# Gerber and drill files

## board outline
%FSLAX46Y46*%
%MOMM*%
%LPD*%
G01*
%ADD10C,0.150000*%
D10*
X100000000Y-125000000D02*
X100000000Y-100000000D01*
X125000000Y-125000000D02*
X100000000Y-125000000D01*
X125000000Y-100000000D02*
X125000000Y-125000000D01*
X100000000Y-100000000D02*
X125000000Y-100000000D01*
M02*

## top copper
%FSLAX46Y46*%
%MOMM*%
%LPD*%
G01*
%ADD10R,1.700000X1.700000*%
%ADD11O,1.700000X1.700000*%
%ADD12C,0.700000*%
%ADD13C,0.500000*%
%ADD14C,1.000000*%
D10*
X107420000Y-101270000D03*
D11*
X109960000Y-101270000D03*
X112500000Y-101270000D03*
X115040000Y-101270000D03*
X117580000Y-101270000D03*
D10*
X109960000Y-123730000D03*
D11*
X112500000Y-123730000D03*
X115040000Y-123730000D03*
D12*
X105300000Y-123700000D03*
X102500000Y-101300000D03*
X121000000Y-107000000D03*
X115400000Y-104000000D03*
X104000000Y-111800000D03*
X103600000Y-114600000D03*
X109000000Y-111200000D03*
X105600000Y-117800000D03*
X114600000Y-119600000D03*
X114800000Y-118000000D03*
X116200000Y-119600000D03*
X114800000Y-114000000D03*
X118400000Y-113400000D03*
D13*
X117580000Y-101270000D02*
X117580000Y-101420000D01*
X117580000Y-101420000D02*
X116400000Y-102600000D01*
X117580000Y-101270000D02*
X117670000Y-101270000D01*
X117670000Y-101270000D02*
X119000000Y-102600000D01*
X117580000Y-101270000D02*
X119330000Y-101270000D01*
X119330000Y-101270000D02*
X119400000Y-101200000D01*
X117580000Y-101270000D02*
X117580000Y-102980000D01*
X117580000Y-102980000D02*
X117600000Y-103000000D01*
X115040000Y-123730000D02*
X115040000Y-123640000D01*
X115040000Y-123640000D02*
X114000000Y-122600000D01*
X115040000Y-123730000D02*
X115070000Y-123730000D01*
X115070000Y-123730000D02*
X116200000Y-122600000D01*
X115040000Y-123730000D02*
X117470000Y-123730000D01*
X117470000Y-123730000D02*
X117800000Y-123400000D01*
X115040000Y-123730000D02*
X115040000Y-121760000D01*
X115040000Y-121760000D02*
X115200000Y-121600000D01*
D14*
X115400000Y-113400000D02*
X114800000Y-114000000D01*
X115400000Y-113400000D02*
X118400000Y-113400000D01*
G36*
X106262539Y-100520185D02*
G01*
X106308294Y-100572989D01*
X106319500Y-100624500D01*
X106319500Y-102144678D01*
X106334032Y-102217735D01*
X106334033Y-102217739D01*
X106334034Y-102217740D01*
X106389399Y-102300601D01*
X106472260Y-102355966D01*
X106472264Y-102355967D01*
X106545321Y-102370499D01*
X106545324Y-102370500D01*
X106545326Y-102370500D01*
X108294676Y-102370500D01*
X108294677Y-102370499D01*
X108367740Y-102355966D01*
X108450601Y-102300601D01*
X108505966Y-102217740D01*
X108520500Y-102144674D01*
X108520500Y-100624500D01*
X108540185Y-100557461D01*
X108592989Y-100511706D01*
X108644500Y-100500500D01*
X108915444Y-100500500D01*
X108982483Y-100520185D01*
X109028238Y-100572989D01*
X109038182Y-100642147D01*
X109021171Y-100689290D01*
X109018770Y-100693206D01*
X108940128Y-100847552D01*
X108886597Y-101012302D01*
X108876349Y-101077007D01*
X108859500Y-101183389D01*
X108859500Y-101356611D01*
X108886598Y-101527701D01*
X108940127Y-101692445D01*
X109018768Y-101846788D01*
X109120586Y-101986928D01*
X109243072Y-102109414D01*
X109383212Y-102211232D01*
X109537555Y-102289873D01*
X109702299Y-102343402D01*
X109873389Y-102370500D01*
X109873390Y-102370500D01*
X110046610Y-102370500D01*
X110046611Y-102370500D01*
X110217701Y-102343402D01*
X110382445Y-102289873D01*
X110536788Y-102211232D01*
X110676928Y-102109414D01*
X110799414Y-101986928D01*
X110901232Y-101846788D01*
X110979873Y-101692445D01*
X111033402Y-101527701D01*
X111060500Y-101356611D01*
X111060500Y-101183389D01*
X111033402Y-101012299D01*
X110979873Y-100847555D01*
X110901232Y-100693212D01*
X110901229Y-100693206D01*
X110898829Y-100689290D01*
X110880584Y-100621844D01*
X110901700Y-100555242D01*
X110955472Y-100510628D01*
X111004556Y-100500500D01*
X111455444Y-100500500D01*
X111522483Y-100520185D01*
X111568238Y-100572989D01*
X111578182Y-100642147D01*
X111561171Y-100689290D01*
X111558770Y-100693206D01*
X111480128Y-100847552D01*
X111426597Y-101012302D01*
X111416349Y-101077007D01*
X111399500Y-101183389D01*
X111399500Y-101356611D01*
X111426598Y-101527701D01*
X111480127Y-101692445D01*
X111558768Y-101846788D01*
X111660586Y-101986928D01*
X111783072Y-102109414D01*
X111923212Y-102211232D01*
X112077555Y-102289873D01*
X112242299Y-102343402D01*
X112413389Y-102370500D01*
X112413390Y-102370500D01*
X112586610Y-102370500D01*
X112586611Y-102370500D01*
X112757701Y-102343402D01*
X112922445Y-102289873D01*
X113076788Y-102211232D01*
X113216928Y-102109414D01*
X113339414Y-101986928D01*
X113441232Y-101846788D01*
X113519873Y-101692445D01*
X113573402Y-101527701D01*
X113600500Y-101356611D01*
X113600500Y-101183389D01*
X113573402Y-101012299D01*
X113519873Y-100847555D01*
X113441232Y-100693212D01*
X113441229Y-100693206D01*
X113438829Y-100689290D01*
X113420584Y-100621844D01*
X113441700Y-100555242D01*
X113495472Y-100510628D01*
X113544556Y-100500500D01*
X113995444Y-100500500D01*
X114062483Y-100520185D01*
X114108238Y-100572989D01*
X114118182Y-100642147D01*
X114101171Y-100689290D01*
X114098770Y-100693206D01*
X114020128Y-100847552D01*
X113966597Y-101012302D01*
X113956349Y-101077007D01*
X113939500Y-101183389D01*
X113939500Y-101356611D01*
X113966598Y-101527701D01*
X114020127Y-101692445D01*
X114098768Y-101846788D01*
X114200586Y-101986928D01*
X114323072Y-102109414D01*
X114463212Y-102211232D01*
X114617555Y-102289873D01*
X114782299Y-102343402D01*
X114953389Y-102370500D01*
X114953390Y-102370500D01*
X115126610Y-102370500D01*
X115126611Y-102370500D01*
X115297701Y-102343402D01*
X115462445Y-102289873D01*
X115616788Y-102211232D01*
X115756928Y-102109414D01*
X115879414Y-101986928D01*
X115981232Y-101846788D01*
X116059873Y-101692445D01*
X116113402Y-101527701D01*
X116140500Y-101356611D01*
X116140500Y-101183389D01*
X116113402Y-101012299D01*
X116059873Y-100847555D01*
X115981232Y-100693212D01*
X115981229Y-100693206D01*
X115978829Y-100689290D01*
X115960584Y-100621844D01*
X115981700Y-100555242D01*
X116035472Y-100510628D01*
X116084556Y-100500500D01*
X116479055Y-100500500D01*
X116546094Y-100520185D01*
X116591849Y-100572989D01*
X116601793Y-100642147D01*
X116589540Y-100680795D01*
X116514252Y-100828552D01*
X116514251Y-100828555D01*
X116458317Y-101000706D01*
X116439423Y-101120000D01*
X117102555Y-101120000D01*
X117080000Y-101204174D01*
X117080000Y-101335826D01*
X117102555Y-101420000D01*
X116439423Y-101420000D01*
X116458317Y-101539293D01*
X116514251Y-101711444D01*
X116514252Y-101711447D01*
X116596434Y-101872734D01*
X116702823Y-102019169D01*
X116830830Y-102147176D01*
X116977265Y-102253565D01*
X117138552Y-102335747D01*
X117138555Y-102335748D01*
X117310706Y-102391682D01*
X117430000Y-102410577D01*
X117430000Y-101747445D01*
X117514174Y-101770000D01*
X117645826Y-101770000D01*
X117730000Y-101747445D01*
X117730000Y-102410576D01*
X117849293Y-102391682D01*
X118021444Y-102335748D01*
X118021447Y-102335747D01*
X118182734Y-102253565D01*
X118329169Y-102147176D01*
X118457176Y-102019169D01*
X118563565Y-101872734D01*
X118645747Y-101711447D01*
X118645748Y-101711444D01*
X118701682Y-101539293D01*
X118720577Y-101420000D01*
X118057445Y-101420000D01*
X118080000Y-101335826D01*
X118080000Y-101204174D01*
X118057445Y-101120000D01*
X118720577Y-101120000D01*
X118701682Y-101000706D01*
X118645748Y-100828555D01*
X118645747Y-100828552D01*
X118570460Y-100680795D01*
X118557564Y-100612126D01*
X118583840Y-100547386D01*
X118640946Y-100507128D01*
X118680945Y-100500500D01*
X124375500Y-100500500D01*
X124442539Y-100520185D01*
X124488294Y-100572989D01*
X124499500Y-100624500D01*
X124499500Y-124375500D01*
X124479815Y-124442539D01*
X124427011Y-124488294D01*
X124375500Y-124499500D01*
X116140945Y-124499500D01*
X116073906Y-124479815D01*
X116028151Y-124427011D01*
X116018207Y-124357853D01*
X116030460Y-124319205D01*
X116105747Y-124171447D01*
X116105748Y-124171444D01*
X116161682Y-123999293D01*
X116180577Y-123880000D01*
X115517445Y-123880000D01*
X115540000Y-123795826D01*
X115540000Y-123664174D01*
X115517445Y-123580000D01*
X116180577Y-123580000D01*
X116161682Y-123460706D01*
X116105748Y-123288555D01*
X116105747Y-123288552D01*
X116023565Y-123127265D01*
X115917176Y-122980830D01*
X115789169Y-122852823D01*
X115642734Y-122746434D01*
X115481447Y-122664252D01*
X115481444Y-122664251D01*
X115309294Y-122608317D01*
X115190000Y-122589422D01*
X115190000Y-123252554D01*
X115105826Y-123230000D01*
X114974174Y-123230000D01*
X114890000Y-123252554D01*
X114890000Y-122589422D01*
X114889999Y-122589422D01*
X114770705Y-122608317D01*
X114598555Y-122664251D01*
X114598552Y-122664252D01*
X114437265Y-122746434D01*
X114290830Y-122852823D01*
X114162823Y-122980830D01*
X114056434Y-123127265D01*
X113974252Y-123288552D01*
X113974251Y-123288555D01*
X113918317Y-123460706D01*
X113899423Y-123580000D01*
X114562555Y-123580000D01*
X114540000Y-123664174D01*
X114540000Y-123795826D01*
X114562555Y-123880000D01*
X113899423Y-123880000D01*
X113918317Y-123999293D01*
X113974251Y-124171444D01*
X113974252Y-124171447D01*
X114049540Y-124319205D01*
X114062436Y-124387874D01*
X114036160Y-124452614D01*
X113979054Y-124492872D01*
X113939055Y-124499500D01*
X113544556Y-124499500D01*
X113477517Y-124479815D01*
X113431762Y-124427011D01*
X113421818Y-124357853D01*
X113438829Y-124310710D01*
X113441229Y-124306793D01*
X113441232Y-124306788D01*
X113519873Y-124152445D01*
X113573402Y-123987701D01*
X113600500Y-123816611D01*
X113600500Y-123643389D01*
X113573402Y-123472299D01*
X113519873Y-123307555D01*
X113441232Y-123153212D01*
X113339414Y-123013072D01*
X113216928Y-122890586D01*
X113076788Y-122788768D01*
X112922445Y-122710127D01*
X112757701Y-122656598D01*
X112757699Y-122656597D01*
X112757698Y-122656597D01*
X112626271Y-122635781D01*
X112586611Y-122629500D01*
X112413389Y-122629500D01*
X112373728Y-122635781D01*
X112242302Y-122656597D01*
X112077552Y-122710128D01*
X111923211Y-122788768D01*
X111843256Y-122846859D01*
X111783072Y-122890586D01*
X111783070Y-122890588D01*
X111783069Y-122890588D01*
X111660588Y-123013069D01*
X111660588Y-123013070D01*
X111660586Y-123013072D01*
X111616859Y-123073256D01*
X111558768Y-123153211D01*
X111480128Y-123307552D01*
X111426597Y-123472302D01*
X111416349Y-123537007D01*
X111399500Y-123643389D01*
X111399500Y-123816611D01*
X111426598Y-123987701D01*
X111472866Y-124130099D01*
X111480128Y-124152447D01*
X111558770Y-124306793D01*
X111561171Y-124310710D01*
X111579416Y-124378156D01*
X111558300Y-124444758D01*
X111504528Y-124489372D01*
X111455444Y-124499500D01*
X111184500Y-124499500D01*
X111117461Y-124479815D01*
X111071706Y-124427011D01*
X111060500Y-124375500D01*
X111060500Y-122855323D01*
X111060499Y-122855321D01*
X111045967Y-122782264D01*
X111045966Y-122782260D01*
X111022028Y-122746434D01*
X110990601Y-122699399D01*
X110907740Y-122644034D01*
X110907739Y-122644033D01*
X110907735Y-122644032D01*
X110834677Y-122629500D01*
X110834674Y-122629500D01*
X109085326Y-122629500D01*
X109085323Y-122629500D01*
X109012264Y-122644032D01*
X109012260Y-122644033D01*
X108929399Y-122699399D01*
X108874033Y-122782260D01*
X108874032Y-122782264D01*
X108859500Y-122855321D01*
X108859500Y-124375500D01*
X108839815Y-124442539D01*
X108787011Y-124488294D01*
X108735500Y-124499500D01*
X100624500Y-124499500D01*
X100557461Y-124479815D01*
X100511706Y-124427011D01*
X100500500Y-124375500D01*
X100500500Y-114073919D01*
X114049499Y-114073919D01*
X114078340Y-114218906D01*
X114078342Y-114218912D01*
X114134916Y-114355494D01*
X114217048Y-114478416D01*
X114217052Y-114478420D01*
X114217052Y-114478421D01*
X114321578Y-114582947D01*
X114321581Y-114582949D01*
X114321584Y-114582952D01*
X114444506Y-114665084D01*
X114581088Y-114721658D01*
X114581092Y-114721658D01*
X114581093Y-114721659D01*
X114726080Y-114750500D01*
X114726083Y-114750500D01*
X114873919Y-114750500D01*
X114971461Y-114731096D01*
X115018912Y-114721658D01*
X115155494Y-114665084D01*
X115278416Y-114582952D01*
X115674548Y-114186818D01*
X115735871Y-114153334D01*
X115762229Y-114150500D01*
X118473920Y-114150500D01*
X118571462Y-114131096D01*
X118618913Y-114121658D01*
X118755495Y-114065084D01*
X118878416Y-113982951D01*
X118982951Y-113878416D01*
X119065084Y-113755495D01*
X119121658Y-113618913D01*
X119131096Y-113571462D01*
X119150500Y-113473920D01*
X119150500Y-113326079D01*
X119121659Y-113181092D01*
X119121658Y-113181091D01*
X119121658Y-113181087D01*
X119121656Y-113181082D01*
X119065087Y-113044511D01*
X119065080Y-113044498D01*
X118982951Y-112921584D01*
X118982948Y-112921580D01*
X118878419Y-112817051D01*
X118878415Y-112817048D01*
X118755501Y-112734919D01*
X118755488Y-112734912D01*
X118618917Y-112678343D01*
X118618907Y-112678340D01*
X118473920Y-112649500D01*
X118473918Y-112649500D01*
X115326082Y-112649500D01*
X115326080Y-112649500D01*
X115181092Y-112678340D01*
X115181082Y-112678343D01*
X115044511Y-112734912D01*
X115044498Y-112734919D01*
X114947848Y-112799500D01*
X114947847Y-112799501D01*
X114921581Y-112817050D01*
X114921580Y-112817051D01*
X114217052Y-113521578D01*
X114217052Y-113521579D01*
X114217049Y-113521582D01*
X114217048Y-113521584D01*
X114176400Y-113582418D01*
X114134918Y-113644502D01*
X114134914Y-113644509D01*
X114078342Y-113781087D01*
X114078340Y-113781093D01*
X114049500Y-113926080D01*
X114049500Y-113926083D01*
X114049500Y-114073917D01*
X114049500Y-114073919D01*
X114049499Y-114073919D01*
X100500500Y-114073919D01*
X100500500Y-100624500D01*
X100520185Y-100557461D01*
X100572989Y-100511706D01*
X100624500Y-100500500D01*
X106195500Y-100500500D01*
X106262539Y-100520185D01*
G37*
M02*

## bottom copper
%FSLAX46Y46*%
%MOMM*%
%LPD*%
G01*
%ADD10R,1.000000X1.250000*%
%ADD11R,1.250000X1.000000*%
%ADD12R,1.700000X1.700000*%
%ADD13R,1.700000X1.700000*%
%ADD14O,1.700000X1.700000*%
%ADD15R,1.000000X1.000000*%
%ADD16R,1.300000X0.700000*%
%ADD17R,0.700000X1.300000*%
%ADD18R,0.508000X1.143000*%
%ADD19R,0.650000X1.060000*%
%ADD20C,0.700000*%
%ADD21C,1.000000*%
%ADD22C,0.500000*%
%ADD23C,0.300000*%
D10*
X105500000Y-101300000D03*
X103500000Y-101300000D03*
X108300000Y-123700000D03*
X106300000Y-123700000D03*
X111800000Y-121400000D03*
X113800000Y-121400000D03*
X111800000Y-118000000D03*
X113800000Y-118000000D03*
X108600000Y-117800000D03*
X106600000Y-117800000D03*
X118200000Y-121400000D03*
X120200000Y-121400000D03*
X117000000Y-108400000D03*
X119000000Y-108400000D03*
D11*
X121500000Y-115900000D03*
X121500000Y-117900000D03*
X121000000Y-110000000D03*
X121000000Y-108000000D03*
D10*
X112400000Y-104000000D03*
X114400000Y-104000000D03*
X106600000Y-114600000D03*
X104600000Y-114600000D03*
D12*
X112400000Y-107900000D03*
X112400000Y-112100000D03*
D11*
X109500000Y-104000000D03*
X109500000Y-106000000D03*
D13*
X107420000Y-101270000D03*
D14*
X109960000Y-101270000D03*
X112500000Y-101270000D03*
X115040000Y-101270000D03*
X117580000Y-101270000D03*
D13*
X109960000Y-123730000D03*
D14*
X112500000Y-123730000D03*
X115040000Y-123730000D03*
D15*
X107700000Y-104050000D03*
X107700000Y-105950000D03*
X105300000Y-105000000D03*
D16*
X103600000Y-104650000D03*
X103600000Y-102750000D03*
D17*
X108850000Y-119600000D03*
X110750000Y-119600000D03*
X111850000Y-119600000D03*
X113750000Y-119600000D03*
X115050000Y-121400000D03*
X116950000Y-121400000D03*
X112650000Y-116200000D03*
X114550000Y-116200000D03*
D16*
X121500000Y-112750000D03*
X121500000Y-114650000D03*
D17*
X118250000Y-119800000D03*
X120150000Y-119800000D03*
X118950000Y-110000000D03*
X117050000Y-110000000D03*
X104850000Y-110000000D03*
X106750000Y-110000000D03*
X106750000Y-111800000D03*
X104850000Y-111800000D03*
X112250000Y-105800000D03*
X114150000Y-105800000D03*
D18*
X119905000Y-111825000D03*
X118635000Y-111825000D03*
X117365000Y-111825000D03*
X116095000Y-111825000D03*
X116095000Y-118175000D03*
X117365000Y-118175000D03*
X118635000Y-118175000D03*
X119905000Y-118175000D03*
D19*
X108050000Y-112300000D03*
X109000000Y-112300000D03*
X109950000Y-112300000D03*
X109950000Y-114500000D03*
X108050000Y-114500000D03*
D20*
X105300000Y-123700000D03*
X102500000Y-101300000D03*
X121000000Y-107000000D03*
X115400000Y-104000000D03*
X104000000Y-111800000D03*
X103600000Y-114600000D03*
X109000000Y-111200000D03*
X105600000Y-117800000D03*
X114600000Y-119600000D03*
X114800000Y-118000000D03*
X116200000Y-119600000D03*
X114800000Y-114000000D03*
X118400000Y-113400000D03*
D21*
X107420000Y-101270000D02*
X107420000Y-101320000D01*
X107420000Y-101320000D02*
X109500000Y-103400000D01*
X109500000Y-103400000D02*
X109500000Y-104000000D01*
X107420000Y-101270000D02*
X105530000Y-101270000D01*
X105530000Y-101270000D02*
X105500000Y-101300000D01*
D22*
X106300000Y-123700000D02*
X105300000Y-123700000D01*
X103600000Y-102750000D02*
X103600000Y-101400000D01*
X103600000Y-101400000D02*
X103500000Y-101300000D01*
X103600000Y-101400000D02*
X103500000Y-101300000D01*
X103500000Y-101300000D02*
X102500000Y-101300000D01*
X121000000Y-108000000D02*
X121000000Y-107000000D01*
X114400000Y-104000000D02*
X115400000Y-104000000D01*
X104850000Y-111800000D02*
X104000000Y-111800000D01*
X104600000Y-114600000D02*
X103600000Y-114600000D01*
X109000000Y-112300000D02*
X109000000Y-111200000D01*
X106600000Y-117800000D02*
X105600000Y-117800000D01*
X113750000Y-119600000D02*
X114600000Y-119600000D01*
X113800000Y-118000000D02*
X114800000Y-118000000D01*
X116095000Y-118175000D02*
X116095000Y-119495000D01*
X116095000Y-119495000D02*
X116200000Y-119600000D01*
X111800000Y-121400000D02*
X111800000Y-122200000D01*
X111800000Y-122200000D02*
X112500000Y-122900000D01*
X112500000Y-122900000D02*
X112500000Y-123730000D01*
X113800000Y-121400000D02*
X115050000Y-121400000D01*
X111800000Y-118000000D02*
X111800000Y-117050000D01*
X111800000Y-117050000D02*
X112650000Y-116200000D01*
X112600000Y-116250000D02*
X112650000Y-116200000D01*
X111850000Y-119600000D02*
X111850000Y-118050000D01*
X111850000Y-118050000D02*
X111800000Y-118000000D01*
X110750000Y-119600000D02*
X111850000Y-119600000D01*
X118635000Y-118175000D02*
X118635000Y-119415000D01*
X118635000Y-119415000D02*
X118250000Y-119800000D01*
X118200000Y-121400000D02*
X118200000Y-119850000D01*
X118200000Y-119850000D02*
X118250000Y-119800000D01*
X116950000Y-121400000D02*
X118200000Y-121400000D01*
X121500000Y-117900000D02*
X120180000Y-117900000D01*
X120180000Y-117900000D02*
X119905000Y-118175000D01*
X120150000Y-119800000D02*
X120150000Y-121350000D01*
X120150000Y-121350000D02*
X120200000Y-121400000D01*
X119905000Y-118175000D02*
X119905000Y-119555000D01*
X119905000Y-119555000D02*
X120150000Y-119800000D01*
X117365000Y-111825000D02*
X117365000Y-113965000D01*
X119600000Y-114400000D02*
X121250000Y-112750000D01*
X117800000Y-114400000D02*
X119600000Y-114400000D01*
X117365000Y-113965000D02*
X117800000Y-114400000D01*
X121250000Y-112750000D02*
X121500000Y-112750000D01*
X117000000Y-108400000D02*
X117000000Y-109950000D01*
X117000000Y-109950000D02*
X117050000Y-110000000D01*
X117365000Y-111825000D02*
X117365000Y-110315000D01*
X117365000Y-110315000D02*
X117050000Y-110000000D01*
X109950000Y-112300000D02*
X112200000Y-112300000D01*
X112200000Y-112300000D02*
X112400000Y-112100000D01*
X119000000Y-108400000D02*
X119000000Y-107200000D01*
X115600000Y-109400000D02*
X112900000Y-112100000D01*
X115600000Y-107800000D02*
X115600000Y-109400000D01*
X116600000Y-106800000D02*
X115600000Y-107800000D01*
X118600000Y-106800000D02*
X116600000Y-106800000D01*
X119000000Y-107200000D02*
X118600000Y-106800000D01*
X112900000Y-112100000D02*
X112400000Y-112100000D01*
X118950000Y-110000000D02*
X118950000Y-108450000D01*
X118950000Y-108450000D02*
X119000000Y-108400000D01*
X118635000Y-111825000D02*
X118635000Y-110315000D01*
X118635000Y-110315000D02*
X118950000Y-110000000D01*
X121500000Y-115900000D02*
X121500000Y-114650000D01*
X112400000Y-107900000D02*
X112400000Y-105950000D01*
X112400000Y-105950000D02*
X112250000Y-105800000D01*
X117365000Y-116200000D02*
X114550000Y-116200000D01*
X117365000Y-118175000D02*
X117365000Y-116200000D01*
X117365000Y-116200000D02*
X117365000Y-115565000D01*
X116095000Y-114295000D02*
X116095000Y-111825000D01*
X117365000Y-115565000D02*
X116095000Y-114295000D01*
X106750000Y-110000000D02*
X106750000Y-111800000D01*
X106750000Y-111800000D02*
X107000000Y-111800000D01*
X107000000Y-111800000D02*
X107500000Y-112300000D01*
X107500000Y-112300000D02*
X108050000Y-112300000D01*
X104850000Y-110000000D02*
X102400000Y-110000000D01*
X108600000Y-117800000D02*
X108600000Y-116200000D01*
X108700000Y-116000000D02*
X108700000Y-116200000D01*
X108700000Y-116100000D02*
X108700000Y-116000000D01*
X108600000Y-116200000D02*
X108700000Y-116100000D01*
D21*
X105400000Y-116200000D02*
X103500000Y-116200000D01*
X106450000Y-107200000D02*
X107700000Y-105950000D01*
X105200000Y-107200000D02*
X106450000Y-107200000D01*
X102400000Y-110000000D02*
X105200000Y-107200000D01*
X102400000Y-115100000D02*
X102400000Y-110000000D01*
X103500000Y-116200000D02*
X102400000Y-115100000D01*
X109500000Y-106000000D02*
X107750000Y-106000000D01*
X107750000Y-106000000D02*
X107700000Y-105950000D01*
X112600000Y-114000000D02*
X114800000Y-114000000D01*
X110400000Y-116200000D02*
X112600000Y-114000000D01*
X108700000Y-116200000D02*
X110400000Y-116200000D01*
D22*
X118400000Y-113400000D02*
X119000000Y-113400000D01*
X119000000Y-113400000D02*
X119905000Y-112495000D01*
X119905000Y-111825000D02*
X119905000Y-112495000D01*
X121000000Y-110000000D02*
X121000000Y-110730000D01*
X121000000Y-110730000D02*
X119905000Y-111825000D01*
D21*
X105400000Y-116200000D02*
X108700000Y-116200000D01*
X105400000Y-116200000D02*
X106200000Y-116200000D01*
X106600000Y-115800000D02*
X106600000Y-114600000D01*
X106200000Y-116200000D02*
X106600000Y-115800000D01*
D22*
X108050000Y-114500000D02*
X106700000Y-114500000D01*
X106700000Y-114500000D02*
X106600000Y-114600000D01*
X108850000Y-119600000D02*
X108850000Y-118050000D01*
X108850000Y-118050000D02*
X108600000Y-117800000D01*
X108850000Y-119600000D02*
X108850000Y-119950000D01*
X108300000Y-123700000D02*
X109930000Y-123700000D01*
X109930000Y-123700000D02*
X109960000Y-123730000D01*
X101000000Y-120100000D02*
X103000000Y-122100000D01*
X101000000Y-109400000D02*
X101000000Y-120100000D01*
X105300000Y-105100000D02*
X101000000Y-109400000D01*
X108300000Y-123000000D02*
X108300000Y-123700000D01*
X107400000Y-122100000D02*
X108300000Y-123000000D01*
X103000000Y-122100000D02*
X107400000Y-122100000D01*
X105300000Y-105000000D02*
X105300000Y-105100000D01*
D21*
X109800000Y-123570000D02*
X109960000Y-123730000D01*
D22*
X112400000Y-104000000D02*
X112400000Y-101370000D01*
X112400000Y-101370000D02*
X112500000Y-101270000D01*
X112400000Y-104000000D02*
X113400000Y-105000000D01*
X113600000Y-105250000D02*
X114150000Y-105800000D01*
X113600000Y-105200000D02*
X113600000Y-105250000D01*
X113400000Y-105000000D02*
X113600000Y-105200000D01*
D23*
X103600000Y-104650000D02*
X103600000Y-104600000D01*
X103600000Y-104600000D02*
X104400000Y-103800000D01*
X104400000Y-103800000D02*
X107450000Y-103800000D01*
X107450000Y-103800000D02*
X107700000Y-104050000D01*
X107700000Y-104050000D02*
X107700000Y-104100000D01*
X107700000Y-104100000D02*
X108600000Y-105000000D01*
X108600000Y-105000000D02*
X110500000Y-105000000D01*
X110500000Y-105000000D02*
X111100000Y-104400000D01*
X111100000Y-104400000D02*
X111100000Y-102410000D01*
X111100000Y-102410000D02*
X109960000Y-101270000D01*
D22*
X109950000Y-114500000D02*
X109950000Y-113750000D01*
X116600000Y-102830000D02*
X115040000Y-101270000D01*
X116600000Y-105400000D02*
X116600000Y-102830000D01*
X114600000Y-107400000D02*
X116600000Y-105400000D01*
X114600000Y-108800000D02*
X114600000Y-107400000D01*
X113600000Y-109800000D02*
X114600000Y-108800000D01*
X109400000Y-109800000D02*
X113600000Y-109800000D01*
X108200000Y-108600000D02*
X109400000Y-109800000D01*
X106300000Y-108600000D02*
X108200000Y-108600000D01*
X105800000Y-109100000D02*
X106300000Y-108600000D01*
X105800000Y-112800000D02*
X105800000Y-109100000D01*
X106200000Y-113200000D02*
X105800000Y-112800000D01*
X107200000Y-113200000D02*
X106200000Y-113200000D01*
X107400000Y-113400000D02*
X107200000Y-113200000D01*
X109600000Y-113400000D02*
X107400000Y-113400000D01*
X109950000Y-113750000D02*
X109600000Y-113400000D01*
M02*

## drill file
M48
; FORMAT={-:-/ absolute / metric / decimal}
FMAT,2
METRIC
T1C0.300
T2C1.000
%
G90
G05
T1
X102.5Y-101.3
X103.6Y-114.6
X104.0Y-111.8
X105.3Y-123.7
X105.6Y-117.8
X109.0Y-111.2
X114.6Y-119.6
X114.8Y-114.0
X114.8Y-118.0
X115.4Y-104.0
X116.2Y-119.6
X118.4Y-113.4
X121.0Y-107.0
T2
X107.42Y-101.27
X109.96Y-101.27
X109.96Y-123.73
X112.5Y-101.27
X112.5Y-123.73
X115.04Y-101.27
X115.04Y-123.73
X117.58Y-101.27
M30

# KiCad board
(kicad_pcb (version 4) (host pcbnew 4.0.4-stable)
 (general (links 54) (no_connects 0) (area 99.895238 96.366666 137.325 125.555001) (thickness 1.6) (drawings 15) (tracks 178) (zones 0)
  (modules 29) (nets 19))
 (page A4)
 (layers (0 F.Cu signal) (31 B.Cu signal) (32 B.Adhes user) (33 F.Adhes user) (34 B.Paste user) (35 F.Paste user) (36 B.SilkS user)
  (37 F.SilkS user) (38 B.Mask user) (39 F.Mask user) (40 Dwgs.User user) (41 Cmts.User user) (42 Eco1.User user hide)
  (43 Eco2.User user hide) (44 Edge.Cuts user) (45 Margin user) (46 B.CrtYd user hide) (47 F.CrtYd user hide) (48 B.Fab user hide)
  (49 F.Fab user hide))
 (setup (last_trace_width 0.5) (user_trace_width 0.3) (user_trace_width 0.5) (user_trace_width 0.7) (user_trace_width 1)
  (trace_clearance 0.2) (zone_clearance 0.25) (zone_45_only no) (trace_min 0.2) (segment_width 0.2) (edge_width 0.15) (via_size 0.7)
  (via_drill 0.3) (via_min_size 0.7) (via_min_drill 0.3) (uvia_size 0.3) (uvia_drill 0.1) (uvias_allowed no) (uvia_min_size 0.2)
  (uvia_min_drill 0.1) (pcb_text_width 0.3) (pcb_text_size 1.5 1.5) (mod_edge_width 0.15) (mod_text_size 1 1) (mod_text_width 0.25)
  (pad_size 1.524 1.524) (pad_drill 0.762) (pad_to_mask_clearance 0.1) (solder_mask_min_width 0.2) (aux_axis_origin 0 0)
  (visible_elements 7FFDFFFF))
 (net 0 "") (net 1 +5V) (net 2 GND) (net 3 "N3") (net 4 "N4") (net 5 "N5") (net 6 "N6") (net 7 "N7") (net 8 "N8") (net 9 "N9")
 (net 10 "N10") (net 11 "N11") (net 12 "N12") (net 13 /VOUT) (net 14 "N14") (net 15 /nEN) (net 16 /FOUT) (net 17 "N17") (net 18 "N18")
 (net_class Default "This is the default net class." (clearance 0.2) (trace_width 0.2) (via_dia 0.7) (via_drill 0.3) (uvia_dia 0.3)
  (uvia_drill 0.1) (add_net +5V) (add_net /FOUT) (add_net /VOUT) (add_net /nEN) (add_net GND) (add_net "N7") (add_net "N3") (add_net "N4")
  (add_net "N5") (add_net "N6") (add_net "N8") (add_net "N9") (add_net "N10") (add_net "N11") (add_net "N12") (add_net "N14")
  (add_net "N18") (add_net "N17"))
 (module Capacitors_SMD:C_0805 (layer B.Cu) (at 104.5 101.3 180)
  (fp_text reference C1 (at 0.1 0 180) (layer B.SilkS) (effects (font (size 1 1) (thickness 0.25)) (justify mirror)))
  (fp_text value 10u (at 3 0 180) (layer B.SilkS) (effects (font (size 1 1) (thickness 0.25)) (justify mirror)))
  (pad 1 smd rect (at -1 0 180) (size 1 1.25) (layers B.Cu B.Paste B.Mask) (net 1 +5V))
  (pad 2 smd rect (at 1 0 180) (size 1 1.25) (layers B.Cu B.Paste B.Mask) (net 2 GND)))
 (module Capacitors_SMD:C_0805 (layer B.Cu) (at 107.3 123.7 180)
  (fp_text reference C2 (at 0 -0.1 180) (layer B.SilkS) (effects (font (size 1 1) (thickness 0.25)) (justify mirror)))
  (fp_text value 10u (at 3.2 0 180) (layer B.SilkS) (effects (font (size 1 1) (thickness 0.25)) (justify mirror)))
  (pad 1 smd rect (at -1 0 180) (size 1 1.25) (layers B.Cu B.Paste B.Mask) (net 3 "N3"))
  (pad 2 smd rect (at 1 0 180) (size 1 1.25) (layers B.Cu B.Paste B.Mask) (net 2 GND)))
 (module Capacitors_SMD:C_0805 (layer B.Cu) (at 112.8 121.4)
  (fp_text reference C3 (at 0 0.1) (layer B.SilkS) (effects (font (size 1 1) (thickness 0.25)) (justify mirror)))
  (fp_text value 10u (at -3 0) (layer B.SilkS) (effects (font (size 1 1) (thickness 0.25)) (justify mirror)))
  (pad 1 smd rect (at -1 0) (size 1 1.25) (layers B.Cu B.Paste B.Mask) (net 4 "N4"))
  (pad 2 smd rect (at 1 0) (size 1 1.25) (layers B.Cu B.Paste B.Mask) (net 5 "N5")))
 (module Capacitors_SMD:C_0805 (layer B.Cu) (at 112.8 118)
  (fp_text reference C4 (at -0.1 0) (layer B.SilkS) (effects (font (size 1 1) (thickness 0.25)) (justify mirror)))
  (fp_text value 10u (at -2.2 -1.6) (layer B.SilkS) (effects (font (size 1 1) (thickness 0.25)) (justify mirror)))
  (pad 1 smd rect (at -1 0) (size 1 1.25) (layers B.Cu B.Paste B.Mask) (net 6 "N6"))
  (pad 2 smd rect (at 1 0) (size 1 1.25) (layers B.Cu B.Paste B.Mask) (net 2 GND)))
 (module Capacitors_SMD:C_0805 (layer B.Cu) (at 107.6 117.8 180)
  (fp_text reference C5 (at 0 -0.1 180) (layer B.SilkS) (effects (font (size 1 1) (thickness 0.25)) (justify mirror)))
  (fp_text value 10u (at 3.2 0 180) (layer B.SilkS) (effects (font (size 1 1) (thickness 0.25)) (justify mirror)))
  (pad 1 smd rect (at -1 0 180) (size 1 1.25) (layers B.Cu B.Paste B.Mask) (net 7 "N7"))
  (pad 2 smd rect (at 1 0 180) (size 1 1.25) (layers B.Cu B.Paste B.Mask) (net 2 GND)))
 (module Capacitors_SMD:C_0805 (layer B.Cu) (at 119.2 121.4)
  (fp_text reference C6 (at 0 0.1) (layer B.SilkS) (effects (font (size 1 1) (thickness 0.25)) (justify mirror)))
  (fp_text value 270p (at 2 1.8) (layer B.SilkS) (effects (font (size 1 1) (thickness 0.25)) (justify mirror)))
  (pad 1 smd rect (at -1 0) (size 1 1.25) (layers B.Cu B.Paste B.Mask) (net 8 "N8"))
  (pad 2 smd rect (at 1 0) (size 1 1.25) (layers B.Cu B.Paste B.Mask) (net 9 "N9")))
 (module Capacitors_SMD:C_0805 (layer B.Cu) (at 118 108.4)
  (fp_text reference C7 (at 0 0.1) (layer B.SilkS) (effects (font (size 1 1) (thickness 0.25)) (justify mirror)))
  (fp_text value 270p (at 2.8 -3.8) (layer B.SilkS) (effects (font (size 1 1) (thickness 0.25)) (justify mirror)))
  (pad 1 smd rect (at -1 0) (size 1 1.25) (layers B.Cu B.Paste B.Mask) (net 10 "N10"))
  (pad 2 smd rect (at 1 0) (size 1 1.25) (layers B.Cu B.Paste B.Mask) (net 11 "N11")))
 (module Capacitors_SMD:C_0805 (layer B.Cu) (at 121.5 116.9 270)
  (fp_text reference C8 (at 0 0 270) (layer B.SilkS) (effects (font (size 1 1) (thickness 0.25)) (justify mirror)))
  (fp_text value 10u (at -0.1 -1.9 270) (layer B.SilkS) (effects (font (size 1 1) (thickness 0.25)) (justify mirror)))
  (pad 1 smd rect (at -1 0 270) (size 1 1.25) (layers B.Cu B.Paste B.Mask) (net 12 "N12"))
  (pad 2 smd rect (at 1 0 270) (size 1 1.25) (layers B.Cu B.Paste B.Mask) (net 9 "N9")))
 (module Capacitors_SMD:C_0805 (layer B.Cu) (at 121 109 90)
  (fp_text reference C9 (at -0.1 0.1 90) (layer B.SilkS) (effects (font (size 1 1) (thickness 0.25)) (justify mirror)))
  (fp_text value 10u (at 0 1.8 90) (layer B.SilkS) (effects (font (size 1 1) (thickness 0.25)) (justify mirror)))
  (pad 1 smd rect (at -1 0 90) (size 1 1.25) (layers B.Cu B.Paste B.Mask) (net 7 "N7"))
  (pad 2 smd rect (at 1 0 90) (size 1 1.25) (layers B.Cu B.Paste B.Mask) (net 2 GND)))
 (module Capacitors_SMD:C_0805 (layer B.Cu) (at 113.4 104)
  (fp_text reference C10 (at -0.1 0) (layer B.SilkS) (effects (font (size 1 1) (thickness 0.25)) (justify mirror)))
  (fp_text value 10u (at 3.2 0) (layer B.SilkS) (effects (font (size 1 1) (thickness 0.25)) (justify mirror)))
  (pad 1 smd rect (at -1 0) (size 1 1.25) (layers B.Cu B.Paste B.Mask) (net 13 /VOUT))
  (pad 2 smd rect (at 1 0) (size 1 1.25) (layers B.Cu B.Paste B.Mask) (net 2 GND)))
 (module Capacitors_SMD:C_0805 (layer B.Cu) (at 105.6 114.6 180)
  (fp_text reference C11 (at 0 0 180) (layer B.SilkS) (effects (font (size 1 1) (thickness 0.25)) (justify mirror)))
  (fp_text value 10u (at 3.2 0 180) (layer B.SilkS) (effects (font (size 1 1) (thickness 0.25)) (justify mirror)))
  (pad 1 smd rect (at -1 0 180) (size 1 1.25) (layers B.Cu B.Paste B.Mask) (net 7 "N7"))
  (pad 2 smd rect (at 1 0 180) (size 1 1.25) (layers B.Cu B.Paste B.Mask) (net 2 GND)))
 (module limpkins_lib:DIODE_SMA (layer B.Cu) (at 112.4 110 270)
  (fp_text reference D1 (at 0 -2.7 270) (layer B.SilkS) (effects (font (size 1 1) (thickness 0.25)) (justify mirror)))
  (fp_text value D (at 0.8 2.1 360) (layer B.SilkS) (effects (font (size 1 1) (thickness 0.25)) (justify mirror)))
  (pad 1 smd rect (at -2.1 0 270) (size 1.7 1.7) (layers B.Cu B.Paste B.Mask) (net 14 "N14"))
  (pad 2 smd rect (at 2.1 0 270) (size 1.7 1.7) (layers B.Cu B.Paste B.Mask) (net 11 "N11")))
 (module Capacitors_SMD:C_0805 (layer B.Cu) (at 109.5 105 270)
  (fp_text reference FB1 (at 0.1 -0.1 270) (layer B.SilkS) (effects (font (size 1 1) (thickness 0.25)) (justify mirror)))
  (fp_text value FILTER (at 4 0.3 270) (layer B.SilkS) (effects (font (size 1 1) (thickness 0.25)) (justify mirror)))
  (pad 1 smd rect (at -1 0 270) (size 1 1.25) (layers B.Cu B.Paste B.Mask) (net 1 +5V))
  (pad 2 smd rect (at 1 0 270) (size 1 1.25) (layers B.Cu B.Paste B.Mask) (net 7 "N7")))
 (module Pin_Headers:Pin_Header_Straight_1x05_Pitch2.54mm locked (layer F.Cu) (at 107.42 101.27 90)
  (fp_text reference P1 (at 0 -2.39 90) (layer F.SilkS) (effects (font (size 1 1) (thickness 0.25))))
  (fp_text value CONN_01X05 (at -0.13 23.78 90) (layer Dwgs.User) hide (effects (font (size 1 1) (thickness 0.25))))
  (pad 1 thru_hole rect (at 0 0 90) (size 1.7 1.7) (drill 1) (layers *.Cu *.Mask) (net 1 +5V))
  (pad 2 thru_hole oval (at 0 2.54 90) (size 1.7 1.7) (drill 1) (layers *.Cu *.Mask) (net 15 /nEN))
  (pad 3 thru_hole oval (at 0 5.08 90) (size 1.7 1.7) (drill 1) (layers *.Cu *.Mask) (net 13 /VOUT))
  (pad 4 thru_hole oval (at 0 7.62 90) (size 1.7 1.7) (drill 1) (layers *.Cu *.Mask) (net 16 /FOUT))
  (pad 5 thru_hole oval (at 0 10.16 90) (size 1.7 1.7) (drill 1) (layers *.Cu *.Mask) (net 2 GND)))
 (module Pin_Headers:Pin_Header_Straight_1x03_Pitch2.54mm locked (layer F.Cu) (at 109.96 123.73 90)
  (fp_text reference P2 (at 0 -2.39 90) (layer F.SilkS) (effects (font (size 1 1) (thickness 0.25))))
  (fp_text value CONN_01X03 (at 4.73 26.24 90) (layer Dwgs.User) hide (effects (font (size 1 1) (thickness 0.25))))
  (pad 1 thru_hole rect (at 0 0 90) (size 1.7 1.7) (drill 1) (layers *.Cu *.Mask) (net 3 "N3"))
  (pad 2 thru_hole oval (at 0 2.54 90) (size 1.7 1.7) (drill 1) (layers *.Cu *.Mask) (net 4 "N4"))
  (pad 3 thru_hole oval (at 0 5.08 90) (size 1.7 1.7) (drill 1) (layers *.Cu *.Mask) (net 2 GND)))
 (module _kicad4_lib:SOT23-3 (layer B.Cu) (at 106.5 105 270)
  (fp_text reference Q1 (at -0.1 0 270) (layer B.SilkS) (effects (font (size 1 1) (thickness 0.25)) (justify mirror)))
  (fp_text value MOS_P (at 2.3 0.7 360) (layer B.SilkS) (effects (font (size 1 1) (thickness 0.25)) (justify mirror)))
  (pad 1 smd rect (at -0.95 -1.2 270) (size 1 1) (layers B.Cu B.Paste B.Mask) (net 15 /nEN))
  (pad 2 smd rect (at 0.95 -1.2 270) (size 1 1) (layers B.Cu B.Paste B.Mask) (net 7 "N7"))
  (pad 3 smd rect (at 0 1.2 270) (size 1 1) (layers B.Cu B.Paste B.Mask) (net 3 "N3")))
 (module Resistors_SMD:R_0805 (layer B.Cu) (at 103.6 103.7 90)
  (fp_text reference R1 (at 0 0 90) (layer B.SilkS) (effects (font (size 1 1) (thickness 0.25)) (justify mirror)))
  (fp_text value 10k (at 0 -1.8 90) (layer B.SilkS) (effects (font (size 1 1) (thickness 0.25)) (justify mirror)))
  (pad 1 smd rect (at -0.95 0 90) (size 0.7 1.3) (layers B.Cu B.Paste B.Mask) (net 15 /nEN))
  (pad 2 smd rect (at 0.95 0 90) (size 0.7 1.3) (layers B.Cu B.Paste B.Mask) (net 2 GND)))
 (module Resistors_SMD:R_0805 (layer B.Cu) (at 109.8 119.6)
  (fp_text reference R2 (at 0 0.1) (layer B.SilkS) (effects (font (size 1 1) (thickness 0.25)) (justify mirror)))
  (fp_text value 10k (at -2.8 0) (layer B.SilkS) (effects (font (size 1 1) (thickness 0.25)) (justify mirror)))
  (pad 1 smd rect (at -0.95 0) (size 0.7 1.3) (layers B.Cu B.Paste B.Mask) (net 7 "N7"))
  (pad 2 smd rect (at 0.95 0) (size 0.7 1.3) (layers B.Cu B.Paste B.Mask) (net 6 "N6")))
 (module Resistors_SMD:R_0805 (layer B.Cu) (at 112.8 119.6)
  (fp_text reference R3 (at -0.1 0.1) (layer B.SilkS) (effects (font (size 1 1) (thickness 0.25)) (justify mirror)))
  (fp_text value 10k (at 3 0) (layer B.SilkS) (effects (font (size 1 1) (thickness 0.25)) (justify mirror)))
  (pad 1 smd rect (at -0.95 0) (size 0.7 1.3) (layers B.Cu B.Paste B.Mask) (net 6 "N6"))
  (pad 2 smd rect (at 0.95 0) (size 0.7 1.3) (layers B.Cu B.Paste B.Mask) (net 2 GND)))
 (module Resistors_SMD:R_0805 (layer B.Cu) (at 116 121.4)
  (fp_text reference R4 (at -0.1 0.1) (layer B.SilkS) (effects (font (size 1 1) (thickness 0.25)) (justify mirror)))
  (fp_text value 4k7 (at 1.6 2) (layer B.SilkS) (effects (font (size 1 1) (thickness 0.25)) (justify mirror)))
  (pad 1 smd rect (at -0.95 0) (size 0.7 1.3) (layers B.Cu B.Paste B.Mask) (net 5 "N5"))
  (pad 2 smd rect (at 0.95 0) (size 0.7 1.3) (layers B.Cu B.Paste B.Mask) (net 8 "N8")))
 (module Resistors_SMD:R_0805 (layer B.Cu) (at 113.6 116.2)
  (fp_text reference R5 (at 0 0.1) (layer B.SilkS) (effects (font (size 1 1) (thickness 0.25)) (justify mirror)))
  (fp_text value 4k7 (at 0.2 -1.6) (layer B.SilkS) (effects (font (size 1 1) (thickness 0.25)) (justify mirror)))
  (pad 1 smd rect (at -0.95 0) (size 0.7 1.3) (layers B.Cu B.Paste B.Mask) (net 6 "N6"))
  (pad 2 smd rect (at 0.95 0) (size 0.7 1.3) (layers B.Cu B.Paste B.Mask) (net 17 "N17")))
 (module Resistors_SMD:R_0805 (layer B.Cu) (at 121.5 113.7 270)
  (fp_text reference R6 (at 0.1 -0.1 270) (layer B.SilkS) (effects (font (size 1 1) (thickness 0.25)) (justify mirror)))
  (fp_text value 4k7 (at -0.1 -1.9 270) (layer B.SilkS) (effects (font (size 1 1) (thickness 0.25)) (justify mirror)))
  (pad 1 smd rect (at -0.95 0 270) (size 0.7 1.3) (layers B.Cu B.Paste B.Mask) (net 10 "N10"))
  (pad 2 smd rect (at 0.95 0 270) (size 0.7 1.3) (layers B.Cu B.Paste B.Mask) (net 12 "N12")))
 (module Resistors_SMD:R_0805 (layer B.Cu) (at 119.2 119.8)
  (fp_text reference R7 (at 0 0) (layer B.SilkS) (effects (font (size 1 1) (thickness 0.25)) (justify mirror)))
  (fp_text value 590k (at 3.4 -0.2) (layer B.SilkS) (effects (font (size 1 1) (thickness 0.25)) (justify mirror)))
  (pad 1 smd rect (at -0.95 0) (size 0.7 1.3) (layers B.Cu B.Paste B.Mask) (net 8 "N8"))
  (pad 2 smd rect (at 0.95 0) (size 0.7 1.3) (layers B.Cu B.Paste B.Mask) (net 9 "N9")))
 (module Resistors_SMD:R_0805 (layer B.Cu) (at 118 110 180)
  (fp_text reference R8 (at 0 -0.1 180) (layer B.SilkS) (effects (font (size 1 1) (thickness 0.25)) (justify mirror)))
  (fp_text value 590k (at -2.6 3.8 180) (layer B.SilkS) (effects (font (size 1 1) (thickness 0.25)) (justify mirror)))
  (pad 1 smd rect (at -0.95 0 180) (size 0.7 1.3) (layers B.Cu B.Paste B.Mask) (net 11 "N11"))
  (pad 2 smd rect (at 0.95 0 180) (size 0.7 1.3) (layers B.Cu B.Paste B.Mask) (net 10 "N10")))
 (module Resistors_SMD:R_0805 (layer B.Cu) (at 105.8 110)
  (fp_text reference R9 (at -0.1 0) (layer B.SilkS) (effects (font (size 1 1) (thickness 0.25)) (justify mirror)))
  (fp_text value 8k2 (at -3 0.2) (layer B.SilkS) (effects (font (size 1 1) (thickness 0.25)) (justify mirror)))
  (pad 1 smd rect (at -0.95 0) (size 0.7 1.3) (layers B.Cu B.Paste B.Mask) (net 7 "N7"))
  (pad 2 smd rect (at 0.95 0) (size 0.7 1.3) (layers B.Cu B.Paste B.Mask) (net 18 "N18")))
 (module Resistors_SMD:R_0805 (layer B.Cu) (at 105.8 111.8 180)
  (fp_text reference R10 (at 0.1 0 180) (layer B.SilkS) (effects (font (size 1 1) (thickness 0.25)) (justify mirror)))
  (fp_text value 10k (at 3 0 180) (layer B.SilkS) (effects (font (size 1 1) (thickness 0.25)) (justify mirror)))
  (pad 1 smd rect (at -0.95 0 180) (size 0.7 1.3) (layers B.Cu B.Paste B.Mask) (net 18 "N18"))
  (pad 2 smd rect (at 0.95 0 180) (size 0.7 1.3) (layers B.Cu B.Paste B.Mask) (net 2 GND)))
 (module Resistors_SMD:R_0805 (layer B.Cu) (at 113.2 105.8)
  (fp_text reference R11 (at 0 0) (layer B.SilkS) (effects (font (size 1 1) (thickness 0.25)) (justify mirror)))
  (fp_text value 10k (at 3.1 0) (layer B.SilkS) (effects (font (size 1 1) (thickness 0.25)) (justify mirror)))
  (pad 1 smd rect (at -0.95 0) (size 0.7 1.3) (layers B.Cu B.Paste B.Mask) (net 14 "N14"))
  (pad 2 smd rect (at 0.95 0) (size 0.7 1.3) (layers B.Cu B.Paste B.Mask) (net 13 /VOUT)))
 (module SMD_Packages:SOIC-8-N (layer B.Cu) (at 118 115 180)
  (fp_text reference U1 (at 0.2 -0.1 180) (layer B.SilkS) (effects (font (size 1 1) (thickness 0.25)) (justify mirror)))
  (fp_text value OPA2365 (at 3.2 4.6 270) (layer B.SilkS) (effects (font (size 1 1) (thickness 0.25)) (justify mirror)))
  (pad 8 smd rect (at -1.905 3.175 180) (size 0.508 1.143) (layers B.Cu B.Paste B.Mask) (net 7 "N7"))
  (pad 7 smd rect (at -0.635 3.175 180) (size 0.508 1.143) (layers B.Cu B.Paste B.Mask) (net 11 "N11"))
  (pad 6 smd rect (at 0.635 3.175 180) (size 0.508 1.143) (layers B.Cu B.Paste B.Mask) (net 10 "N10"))
  (pad 5 smd rect (at 1.905 3.175 180) (size 0.508 1.143) (layers B.Cu B.Paste B.Mask) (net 17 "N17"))
  (pad 4 smd rect (at 1.905 -3.175 180) (size 0.508 1.143) (layers B.Cu B.Paste B.Mask) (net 2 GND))
  (pad 3 smd rect (at 0.635 -3.175 180) (size 0.508 1.143) (layers B.Cu B.Paste B.Mask) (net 17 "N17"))
  (pad 2 smd rect (at -0.635 -3.175 180) (size 0.508 1.143) (layers B.Cu B.Paste B.Mask) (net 8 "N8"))
  (pad 1 smd rect (at -1.905 -3.175 180) (size 0.508 1.143) (layers B.Cu B.Paste B.Mask) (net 9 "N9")))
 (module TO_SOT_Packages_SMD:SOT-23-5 (layer B.Cu) (at 109 113.4 270)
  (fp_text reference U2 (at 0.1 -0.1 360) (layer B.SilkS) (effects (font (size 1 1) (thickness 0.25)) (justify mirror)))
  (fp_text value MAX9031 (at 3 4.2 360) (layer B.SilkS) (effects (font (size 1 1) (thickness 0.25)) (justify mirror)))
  (pad 1 smd rect (at -1.1 0.95 270) (size 1.06 0.65) (layers B.Cu B.Paste B.Mask) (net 18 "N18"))
  (pad 2 smd rect (at -1.1 0 270) (size 1.06 0.65) (layers B.Cu B.Paste B.Mask) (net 2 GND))
  (pad 3 smd rect (at -1.1 -0.95 270) (size 1.06 0.65) (layers B.Cu B.Paste B.Mask) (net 11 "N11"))
  (pad 4 smd rect (at 1.1 -0.95 270) (size 1.06 0.65) (layers B.Cu B.Paste B.Mask) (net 16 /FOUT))
  (pad 5 smd rect (at 1.1 0.95 270) (size 1.06 0.65) (layers B.Cu B.Paste B.Mask) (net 7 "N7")))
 (gr_line (start 100 125) (end 100 100) (angle 90) (layer Edge.Cuts) (width 0.15))
 (gr_line (start 125 125) (end 100 125) (angle 90) (layer Edge.Cuts) (width 0.15))
 (gr_line (start 125 100) (end 125 125) (angle 90) (layer Edge.Cuts) (width 0.15))
 (gr_line (start 100 100) (end 125 100) (angle 90) (layer Edge.Cuts) (width 0.15))
 (segment (start 107.42 101.27) (end 107.42 101.32) (width 1) (layer B.Cu) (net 1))
 (segment (start 107.42 101.32) (end 109.5 103.4) (width 1) (layer B.Cu) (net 1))
 (segment (start 109.5 103.4) (end 109.5 104) (width 1) (layer B.Cu) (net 1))
 (segment (start 107.42 101.27) (end 105.53 101.27) (width 1) (layer B.Cu) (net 1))
 (segment (start 105.53 101.27) (end 105.5 101.3) (width 1) (layer B.Cu) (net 1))
 (segment (start 106.3 123.7) (end 105.3 123.7) (width 0.5) (layer B.Cu) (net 2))
 (via (at 105.3 123.7) (size 0.7) (drill 0.3) (layers F.Cu B.Cu) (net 2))
 (segment (start 103.6 102.75) (end 103.6 101.4) (width 0.5) (layer B.Cu) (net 2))
 (segment (start 103.6 101.4) (end 103.5 101.3) (width 0.5) (layer B.Cu) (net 2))
 (segment (start 103.6 101.4) (end 103.5 101.3) (width 0.5) (layer B.Cu) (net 2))
 (segment (start 103.5 101.3) (end 102.5 101.3) (width 0.5) (layer B.Cu) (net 2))
 (via (at 102.5 101.3) (size 0.7) (drill 0.3) (layers F.Cu B.Cu) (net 2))
 (segment (start 117.58 101.27) (end 117.58 101.42) (width 0.5) (layer F.Cu) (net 2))
 (segment (start 117.58 101.42) (end 116.4 102.6) (width 0.5) (layer F.Cu) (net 2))
 (segment (start 117.58 101.27) (end 117.67 101.27) (width 0.5) (layer F.Cu) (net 2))
 (segment (start 117.67 101.27) (end 119 102.6) (width 0.5) (layer F.Cu) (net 2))
 (segment (start 117.58 101.27) (end 119.33 101.27) (width 0.5) (layer F.Cu) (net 2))
 (segment (start 119.33 101.27) (end 119.4 101.2) (width 0.5) (layer F.Cu) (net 2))
 (segment (start 117.58 101.27) (end 117.58 102.98) (width 0.5) (layer F.Cu) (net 2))
 (segment (start 117.58 102.98) (end 117.6 103) (width 0.5) (layer F.Cu) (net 2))
 (segment (start 115.04 123.73) (end 115.04 123.64) (width 0.5) (layer F.Cu) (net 2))
 (segment (start 115.04 123.64) (end 114 122.6) (width 0.5) (layer F.Cu) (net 2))
 (segment (start 115.04 123.73) (end 115.07 123.73) (width 0.5) (layer F.Cu) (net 2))
 (segment (start 115.07 123.73) (end 116.2 122.6) (width 0.5) (layer F.Cu) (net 2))
 (segment (start 115.04 123.73) (end 117.47 123.73) (width 0.5) (layer F.Cu) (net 2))
 (segment (start 117.47 123.73) (end 117.8 123.4) (width 0.5) (layer F.Cu) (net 2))
 (segment (start 115.04 123.73) (end 115.04 121.76) (width 0.5) (layer F.Cu) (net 2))
 (segment (start 115.04 121.76) (end 115.2 121.6) (width 0.5) (layer F.Cu) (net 2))
 (segment (start 121 108) (end 121 107) (width 0.5) (layer B.Cu) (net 2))
 (via (at 121 107) (size 0.7) (drill 0.3) (layers F.Cu B.Cu) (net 2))
 (segment (start 114.4 104) (end 115.4 104) (width 0.5) (layer B.Cu) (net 2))
 (via (at 115.4 104) (size 0.7) (drill 0.3) (layers F.Cu B.Cu) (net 2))
 (segment (start 104.85 111.8) (end 104 111.8) (width 0.5) (layer B.Cu) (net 2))
 (via (at 104 111.8) (size 0.7) (drill 0.3) (layers F.Cu B.Cu) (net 2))
 (segment (start 104.6 114.6) (end 103.6 114.6) (width 0.5) (layer B.Cu) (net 2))
 (via (at 103.6 114.6) (size 0.7) (drill 0.3) (layers F.Cu B.Cu) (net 2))
 (segment (start 109 112.3) (end 109 111.2) (width 0.5) (layer B.Cu) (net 2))
 (via (at 109 111.2) (size 0.7) (drill 0.3) (layers F.Cu B.Cu) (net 2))
 (segment (start 106.6 117.8) (end 105.6 117.8) (width 0.5) (layer B.Cu) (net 2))
 (via (at 105.6 117.8) (size 0.7) (drill 0.3) (layers F.Cu B.Cu) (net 2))
 (segment (start 113.75 119.6) (end 114.6 119.6) (width 0.5) (layer B.Cu) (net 2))
 (via (at 114.6 119.6) (size 0.7) (drill 0.3) (layers F.Cu B.Cu) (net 2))
 (segment (start 113.8 118) (end 114.8 118) (width 0.5) (layer B.Cu) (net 2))
 (via (at 114.8 118) (size 0.7) (drill 0.3) (layers F.Cu B.Cu) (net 2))
 (segment (start 116.095 118.175) (end 116.095 119.495) (width 0.5) (layer B.Cu) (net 2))
 (via (at 116.2 119.6) (size 0.7) (drill 0.3) (layers F.Cu B.Cu) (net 2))
 (segment (start 116.095 119.495) (end 116.2 119.6) (width 0.5) (layer B.Cu) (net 2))
 (segment (start 111.8 121.4) (end 111.8 122.2) (width 0.5) (layer B.Cu) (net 4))
 (segment (start 111.8 122.2) (end 112.5 122.9) (width 0.5) (layer B.Cu) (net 4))
 (segment (start 112.5 122.9) (end 112.5 123.73) (width 0.5) (layer B.Cu) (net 4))
 (segment (start 113.8 121.4) (end 115.05 121.4) (width 0.5) (layer B.Cu) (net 5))
 (segment (start 111.8 118) (end 111.8 117.05) (width 0.5) (layer B.Cu) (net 6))
 (segment (start 111.8 117.05) (end 112.65 116.2) (width 0.5) (layer B.Cu) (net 6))
 (segment (start 112.6 116.25) (end 112.65 116.2) (width 0.5) (layer B.Cu) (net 6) (status 30))
 (segment (start 111.85 119.6) (end 111.85 118.05) (width 0.5) (layer B.Cu) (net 6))
 (segment (start 111.85 118.05) (end 111.8 118) (width 0.5) (layer B.Cu) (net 6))
 (segment (start 110.75 119.6) (end 111.85 119.6) (width 0.5) (layer B.Cu) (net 6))
 (segment (start 118.635 118.175) (end 118.635 119.415) (width 0.5) (layer B.Cu) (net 8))
 (segment (start 118.635 119.415) (end 118.25 119.8) (width 0.5) (layer B.Cu) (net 8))
 (segment (start 118.2 121.4) (end 118.2 119.85) (width 0.5) (layer B.Cu) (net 8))
 (segment (start 118.2 119.85) (end 118.25 119.8) (width 0.5) (layer B.Cu) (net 8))
 (segment (start 116.95 121.4) (end 118.2 121.4) (width 0.5) (layer B.Cu) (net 8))
 (segment (start 121.5 117.9) (end 120.18 117.9) (width 0.5) (layer B.Cu) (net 9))
 (segment (start 120.18 117.9) (end 119.905 118.175) (width 0.5) (layer B.Cu) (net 9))
 (segment (start 120.15 119.8) (end 120.15 121.35) (width 0.5) (layer B.Cu) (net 9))
 (segment (start 120.15 121.35) (end 120.2 121.4) (width 0.5) (layer B.Cu) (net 9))
 (segment (start 119.905 118.175) (end 119.905 119.555) (width 0.5) (layer B.Cu) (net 9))
 (segment (start 119.905 119.555) (end 120.15 119.8) (width 0.5) (layer B.Cu) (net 9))
 (segment (start 117.365 111.825) (end 117.365 113.965) (width 0.5) (layer B.Cu) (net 10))
 (segment (start 119.6 114.4) (end 121.25 112.75) (width 0.5) (layer B.Cu) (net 10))
 (segment (start 117.8 114.4) (end 119.6 114.4) (width 0.5) (layer B.Cu) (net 10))
 (segment (start 117.365 113.965) (end 117.8 114.4) (width 0.5) (layer B.Cu) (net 10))
 (segment (start 121.25 112.75) (end 121.5 112.75) (width 0.5) (layer B.Cu) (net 10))
 (segment (start 117 108.4) (end 117 109.95) (width 0.5) (layer B.Cu) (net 10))
 (segment (start 117 109.95) (end 117.05 110) (width 0.5) (layer B.Cu) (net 10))
 (segment (start 117.365 111.825) (end 117.365 110.315) (width 0.5) (layer B.Cu) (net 10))
 (segment (start 117.365 110.315) (end 117.05 110) (width 0.5) (layer B.Cu) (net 10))
 (segment (start 109.95 112.3) (end 112.2 112.3) (width 0.5) (layer B.Cu) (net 11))
 (segment (start 112.2 112.3) (end 112.4 112.1) (width 0.5) (layer B.Cu) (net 11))
 (segment (start 119 108.4) (end 119 107.2) (width 0.5) (layer B.Cu) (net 11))
 (segment (start 115.6 109.4) (end 112.9 112.1) (width 0.5) (layer B.Cu) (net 11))
 (segment (start 115.6 107.8) (end 115.6 109.4) (width 0.5) (layer B.Cu) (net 11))
 (segment (start 116.6 106.8) (end 115.6 107.8) (width 0.5) (layer B.Cu) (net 11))
 (segment (start 118.6 106.8) (end 116.6 106.8) (width 0.5) (layer B.Cu) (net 11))
 (segment (start 119 107.2) (end 118.6 106.8) (width 0.5) (layer B.Cu) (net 11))
 (segment (start 112.9 112.1) (end 112.4 112.1) (width 0.5) (layer B.Cu) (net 11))
 (segment (start 118.95 110) (end 118.95 108.45) (width 0.5) (layer B.Cu) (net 11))
 (segment (start 118.95 108.45) (end 119 108.4) (width 0.5) (layer B.Cu) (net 11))
 (segment (start 118.635 111.825) (end 118.635 110.315) (width 0.5) (layer B.Cu) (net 11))
 (segment (start 118.635 110.315) (end 118.95 110) (width 0.5) (layer B.Cu) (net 11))
 (segment (start 121.5 115.9) (end 121.5 114.65) (width 0.5) (layer B.Cu) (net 12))
 (segment (start 112.4 107.9) (end 112.4 105.95) (width 0.5) (layer B.Cu) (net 14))
 (segment (start 112.4 105.95) (end 112.25 105.8) (width 0.5) (layer B.Cu) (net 14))
 (segment (start 117.365 116.2) (end 114.55 116.2) (width 0.5) (layer B.Cu) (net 17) (status 20))
 (segment (start 117.365 118.175) (end 117.365 116.2) (width 0.5) (layer B.Cu) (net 17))
 (segment (start 117.365 116.2) (end 117.365 115.565) (width 0.5) (layer B.Cu) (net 17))
 (segment (start 116.095 114.295) (end 116.095 111.825) (width 0.5) (layer B.Cu) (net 17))
 (segment (start 117.365 115.565) (end 116.095 114.295) (width 0.5) (layer B.Cu) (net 17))
 (segment (start 106.75 110) (end 106.75 111.8) (width 0.5) (layer B.Cu) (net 18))
 (segment (start 106.75 111.8) (end 107 111.8) (width 0.5) (layer B.Cu) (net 18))
 (segment (start 107 111.8) (end 107.5 112.3) (width 0.5) (layer B.Cu) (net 18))
 (segment (start 107.5 112.3) (end 108.05 112.3) (width 0.5) (layer B.Cu) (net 18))
 (segment (start 104.85 110) (end 102.4 110) (width 0.5) (layer B.Cu) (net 7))
 (segment (start 108.6 117.8) (end 108.6 116.2) (width 0.5) (layer B.Cu) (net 7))
 (segment (start 108.7 116) (end 108.7 116.2) (width 0.5) (layer B.Cu) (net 7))
 (segment (start 108.7 116.1) (end 108.7 116) (width 0.5) (layer B.Cu) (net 7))
 (segment (start 108.6 116.2) (end 108.7 116.1) (width 0.5) (layer B.Cu) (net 7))
 (segment (start 105.4 116.2) (end 103.5 116.2) (width 1) (layer B.Cu) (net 7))
 (segment (start 106.45 107.2) (end 107.7 105.95) (width 1) (layer B.Cu) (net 7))
 (segment (start 105.2 107.2) (end 106.45 107.2) (width 1) (layer B.Cu) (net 7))
 (segment (start 102.4 110) (end 105.2 107.2) (width 1) (layer B.Cu) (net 7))
 (segment (start 102.4 115.1) (end 102.4 110) (width 1) (layer B.Cu) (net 7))
 (segment (start 103.5 116.2) (end 102.4 115.1) (width 1) (layer B.Cu) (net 7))
 (segment (start 109.5 106) (end 107.75 106) (width 1) (layer B.Cu) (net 7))
 (segment (start 107.75 106) (end 107.7 105.95) (width 1) (layer B.Cu) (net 7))
 (via (at 114.8 114) (size 0.7) (drill 0.3) (layers F.Cu B.Cu) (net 7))
 (segment (start 112.6 114) (end 114.8 114) (width 1) (layer B.Cu) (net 7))
 (segment (start 110.4 116.2) (end 112.6 114) (width 1) (layer B.Cu) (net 7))
 (segment (start 108.7 116.2) (end 110.4 116.2) (width 1) (layer B.Cu) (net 7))
 (segment (start 115.4 113.4) (end 114.8 114) (width 1) (layer F.Cu) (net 7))
 (segment (start 115.4 113.4) (end 118.4 113.4) (width 1) (layer F.Cu) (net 7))
 (via (at 118.4 113.4) (size 0.7) (drill 0.3) (layers F.Cu B.Cu) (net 7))
 (segment (start 118.4 113.4) (end 119 113.4) (width 0.5) (layer B.Cu) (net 7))
 (segment (start 119 113.4) (end 119.905 112.495) (width 0.5) (layer B.Cu) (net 7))
 (segment (start 119.905 111.825) (end 119.905 112.495) (width 0.5) (layer B.Cu) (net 7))
 (segment (start 121 110) (end 121 110.73) (width 0.5) (layer B.Cu) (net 7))
 (segment (start 121 110.73) (end 119.905 111.825) (width 0.5) (layer B.Cu) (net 7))
 (segment (start 105.4 116.2) (end 108.7 116.2) (width 1) (layer B.Cu) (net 7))
 (segment (start 105.4 116.2) (end 106.2 116.2) (width 1) (layer B.Cu) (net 7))
 (segment (start 106.6 115.8) (end 106.6 114.6) (width 1) (layer B.Cu) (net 7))
 (segment (start 106.2 116.2) (end 106.6 115.8) (width 1) (layer B.Cu) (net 7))
 (segment (start 108.05 114.5) (end 106.7 114.5) (width 0.5) (layer B.Cu) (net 7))
 (segment (start 106.7 114.5) (end 106.6 114.6) (width 0.5) (layer B.Cu) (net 7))
 (segment (start 108.85 119.6) (end 108.85 118.05) (width 0.5) (layer B.Cu) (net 7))
 (segment (start 108.85 118.05) (end 108.6 117.8) (width 0.5) (layer B.Cu) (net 7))
 (segment (start 108.85 119.6) (end 108.85 119.95) (width 0.5) (layer B.Cu) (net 7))
 (segment (start 108.3 123.7) (end 109.93 123.7) (width 0.5) (layer B.Cu) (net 3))
 (segment (start 109.93 123.7) (end 109.96 123.73) (width 0.5) (layer B.Cu) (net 3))
 (segment (start 101 120.1) (end 103 122.1) (width 0.5) (layer B.Cu) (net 3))
 (segment (start 101 109.4) (end 101 120.1) (width 0.5) (layer B.Cu) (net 3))
 (segment (start 105.3 105.1) (end 101 109.4) (width 0.5) (layer B.Cu) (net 3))
 (segment (start 108.3 123) (end 108.3 123.7) (width 0.5) (layer B.Cu) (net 3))
 (segment (start 107.4 122.1) (end 108.3 123) (width 0.5) (layer B.Cu) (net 3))
 (segment (start 103 122.1) (end 107.4 122.1) (width 0.5) (layer B.Cu) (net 3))
 (segment (start 105.3 105) (end 105.3 105.1) (width 0.5) (layer B.Cu) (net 3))
 (segment (start 109.8 123.57) (end 109.96 123.73) (width 1) (layer B.Cu) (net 3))
 (segment (start 112.4 104) (end 112.4 101.37) (width 0.5) (layer B.Cu) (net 13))
 (segment (start 112.4 101.37) (end 112.5 101.27) (width 0.5) (layer B.Cu) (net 13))
 (segment (start 112.4 104) (end 113.4 105) (width 0.5) (layer B.Cu) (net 13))
 (segment (start 113.6 105.25) (end 114.15 105.8) (width 0.5) (layer B.Cu) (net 13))
 (segment (start 113.6 105.2) (end 113.6 105.25) (width 0.5) (layer B.Cu) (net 13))
 (segment (start 113.4 105) (end 113.6 105.2) (width 0.5) (layer B.Cu) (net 13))
 (segment (start 103.6 104.65) (end 103.6 104.6) (width 0.3) (layer B.Cu) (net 15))
 (segment (start 103.6 104.6) (end 104.4 103.8) (width 0.3) (layer B.Cu) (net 15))
 (segment (start 104.4 103.8) (end 107.45 103.8) (width 0.3) (layer B.Cu) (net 15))
 (segment (start 107.45 103.8) (end 107.7 104.05) (width 0.3) (layer B.Cu) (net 15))
 (segment (start 107.7 104.05) (end 107.7 104.1) (width 0.3) (layer B.Cu) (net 15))
 (segment (start 107.7 104.1) (end 108.6 105) (width 0.3) (layer B.Cu) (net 15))
 (segment (start 108.6 105) (end 110.5 105) (width 0.3) (layer B.Cu) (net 15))
 (segment (start 110.5 105) (end 111.1 104.4) (width 0.3) (layer B.Cu) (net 15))
 (segment (start 111.1 104.4) (end 111.1 102.41) (width 0.3) (layer B.Cu) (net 15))
 (segment (start 111.1 102.41) (end 109.96 101.27) (width 0.3) (layer B.Cu) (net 15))
 (segment (start 109.95 114.5) (end 109.95 113.75) (width 0.5) (layer B.Cu) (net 16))
 (segment (start 116.6 102.83) (end 115.04 101.27) (width 0.5) (layer B.Cu) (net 16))
 (segment (start 116.6 105.4) (end 116.6 102.83) (width 0.5) (layer B.Cu) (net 16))
 (segment (start 114.6 107.4) (end 116.6 105.4) (width 0.5) (layer B.Cu) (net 16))
 (segment (start 114.6 108.8) (end 114.6 107.4) (width 0.5) (layer B.Cu) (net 16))
 (segment (start 113.6 109.8) (end 114.6 108.8) (width 0.5) (layer B.Cu) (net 16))
 (segment (start 109.4 109.8) (end 113.6 109.8) (width 0.5) (layer B.Cu) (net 16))
 (segment (start 108.2 108.6) (end 109.4 109.8) (width 0.5) (layer B.Cu) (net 16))
 (segment (start 106.3 108.6) (end 108.2 108.6) (width 0.5) (layer B.Cu) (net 16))
 (segment (start 105.8 109.1) (end 106.3 108.6) (width 0.5) (layer B.Cu) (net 16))
 (segment (start 105.8 112.8) (end 105.8 109.1) (width 0.5) (layer B.Cu) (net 16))
 (segment (start 106.2 113.2) (end 105.8 112.8) (width 0.5) (layer B.Cu) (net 16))
 (segment (start 107.2 113.2) (end 106.2 113.2) (width 0.5) (layer B.Cu) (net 16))
 (segment (start 107.4 113.4) (end 107.2 113.2) (width 0.5) (layer B.Cu) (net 16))
 (segment (start 109.6 113.4) (end 107.4 113.4) (width 0.5) (layer B.Cu) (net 16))
 (segment (start 109.95 113.75) (end 109.6 113.4) (width 0.5) (layer B.Cu) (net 16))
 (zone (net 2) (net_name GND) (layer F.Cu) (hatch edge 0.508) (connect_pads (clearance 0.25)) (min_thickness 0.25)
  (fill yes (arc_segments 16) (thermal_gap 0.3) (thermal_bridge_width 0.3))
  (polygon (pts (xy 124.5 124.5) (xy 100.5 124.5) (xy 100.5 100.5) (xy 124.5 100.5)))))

